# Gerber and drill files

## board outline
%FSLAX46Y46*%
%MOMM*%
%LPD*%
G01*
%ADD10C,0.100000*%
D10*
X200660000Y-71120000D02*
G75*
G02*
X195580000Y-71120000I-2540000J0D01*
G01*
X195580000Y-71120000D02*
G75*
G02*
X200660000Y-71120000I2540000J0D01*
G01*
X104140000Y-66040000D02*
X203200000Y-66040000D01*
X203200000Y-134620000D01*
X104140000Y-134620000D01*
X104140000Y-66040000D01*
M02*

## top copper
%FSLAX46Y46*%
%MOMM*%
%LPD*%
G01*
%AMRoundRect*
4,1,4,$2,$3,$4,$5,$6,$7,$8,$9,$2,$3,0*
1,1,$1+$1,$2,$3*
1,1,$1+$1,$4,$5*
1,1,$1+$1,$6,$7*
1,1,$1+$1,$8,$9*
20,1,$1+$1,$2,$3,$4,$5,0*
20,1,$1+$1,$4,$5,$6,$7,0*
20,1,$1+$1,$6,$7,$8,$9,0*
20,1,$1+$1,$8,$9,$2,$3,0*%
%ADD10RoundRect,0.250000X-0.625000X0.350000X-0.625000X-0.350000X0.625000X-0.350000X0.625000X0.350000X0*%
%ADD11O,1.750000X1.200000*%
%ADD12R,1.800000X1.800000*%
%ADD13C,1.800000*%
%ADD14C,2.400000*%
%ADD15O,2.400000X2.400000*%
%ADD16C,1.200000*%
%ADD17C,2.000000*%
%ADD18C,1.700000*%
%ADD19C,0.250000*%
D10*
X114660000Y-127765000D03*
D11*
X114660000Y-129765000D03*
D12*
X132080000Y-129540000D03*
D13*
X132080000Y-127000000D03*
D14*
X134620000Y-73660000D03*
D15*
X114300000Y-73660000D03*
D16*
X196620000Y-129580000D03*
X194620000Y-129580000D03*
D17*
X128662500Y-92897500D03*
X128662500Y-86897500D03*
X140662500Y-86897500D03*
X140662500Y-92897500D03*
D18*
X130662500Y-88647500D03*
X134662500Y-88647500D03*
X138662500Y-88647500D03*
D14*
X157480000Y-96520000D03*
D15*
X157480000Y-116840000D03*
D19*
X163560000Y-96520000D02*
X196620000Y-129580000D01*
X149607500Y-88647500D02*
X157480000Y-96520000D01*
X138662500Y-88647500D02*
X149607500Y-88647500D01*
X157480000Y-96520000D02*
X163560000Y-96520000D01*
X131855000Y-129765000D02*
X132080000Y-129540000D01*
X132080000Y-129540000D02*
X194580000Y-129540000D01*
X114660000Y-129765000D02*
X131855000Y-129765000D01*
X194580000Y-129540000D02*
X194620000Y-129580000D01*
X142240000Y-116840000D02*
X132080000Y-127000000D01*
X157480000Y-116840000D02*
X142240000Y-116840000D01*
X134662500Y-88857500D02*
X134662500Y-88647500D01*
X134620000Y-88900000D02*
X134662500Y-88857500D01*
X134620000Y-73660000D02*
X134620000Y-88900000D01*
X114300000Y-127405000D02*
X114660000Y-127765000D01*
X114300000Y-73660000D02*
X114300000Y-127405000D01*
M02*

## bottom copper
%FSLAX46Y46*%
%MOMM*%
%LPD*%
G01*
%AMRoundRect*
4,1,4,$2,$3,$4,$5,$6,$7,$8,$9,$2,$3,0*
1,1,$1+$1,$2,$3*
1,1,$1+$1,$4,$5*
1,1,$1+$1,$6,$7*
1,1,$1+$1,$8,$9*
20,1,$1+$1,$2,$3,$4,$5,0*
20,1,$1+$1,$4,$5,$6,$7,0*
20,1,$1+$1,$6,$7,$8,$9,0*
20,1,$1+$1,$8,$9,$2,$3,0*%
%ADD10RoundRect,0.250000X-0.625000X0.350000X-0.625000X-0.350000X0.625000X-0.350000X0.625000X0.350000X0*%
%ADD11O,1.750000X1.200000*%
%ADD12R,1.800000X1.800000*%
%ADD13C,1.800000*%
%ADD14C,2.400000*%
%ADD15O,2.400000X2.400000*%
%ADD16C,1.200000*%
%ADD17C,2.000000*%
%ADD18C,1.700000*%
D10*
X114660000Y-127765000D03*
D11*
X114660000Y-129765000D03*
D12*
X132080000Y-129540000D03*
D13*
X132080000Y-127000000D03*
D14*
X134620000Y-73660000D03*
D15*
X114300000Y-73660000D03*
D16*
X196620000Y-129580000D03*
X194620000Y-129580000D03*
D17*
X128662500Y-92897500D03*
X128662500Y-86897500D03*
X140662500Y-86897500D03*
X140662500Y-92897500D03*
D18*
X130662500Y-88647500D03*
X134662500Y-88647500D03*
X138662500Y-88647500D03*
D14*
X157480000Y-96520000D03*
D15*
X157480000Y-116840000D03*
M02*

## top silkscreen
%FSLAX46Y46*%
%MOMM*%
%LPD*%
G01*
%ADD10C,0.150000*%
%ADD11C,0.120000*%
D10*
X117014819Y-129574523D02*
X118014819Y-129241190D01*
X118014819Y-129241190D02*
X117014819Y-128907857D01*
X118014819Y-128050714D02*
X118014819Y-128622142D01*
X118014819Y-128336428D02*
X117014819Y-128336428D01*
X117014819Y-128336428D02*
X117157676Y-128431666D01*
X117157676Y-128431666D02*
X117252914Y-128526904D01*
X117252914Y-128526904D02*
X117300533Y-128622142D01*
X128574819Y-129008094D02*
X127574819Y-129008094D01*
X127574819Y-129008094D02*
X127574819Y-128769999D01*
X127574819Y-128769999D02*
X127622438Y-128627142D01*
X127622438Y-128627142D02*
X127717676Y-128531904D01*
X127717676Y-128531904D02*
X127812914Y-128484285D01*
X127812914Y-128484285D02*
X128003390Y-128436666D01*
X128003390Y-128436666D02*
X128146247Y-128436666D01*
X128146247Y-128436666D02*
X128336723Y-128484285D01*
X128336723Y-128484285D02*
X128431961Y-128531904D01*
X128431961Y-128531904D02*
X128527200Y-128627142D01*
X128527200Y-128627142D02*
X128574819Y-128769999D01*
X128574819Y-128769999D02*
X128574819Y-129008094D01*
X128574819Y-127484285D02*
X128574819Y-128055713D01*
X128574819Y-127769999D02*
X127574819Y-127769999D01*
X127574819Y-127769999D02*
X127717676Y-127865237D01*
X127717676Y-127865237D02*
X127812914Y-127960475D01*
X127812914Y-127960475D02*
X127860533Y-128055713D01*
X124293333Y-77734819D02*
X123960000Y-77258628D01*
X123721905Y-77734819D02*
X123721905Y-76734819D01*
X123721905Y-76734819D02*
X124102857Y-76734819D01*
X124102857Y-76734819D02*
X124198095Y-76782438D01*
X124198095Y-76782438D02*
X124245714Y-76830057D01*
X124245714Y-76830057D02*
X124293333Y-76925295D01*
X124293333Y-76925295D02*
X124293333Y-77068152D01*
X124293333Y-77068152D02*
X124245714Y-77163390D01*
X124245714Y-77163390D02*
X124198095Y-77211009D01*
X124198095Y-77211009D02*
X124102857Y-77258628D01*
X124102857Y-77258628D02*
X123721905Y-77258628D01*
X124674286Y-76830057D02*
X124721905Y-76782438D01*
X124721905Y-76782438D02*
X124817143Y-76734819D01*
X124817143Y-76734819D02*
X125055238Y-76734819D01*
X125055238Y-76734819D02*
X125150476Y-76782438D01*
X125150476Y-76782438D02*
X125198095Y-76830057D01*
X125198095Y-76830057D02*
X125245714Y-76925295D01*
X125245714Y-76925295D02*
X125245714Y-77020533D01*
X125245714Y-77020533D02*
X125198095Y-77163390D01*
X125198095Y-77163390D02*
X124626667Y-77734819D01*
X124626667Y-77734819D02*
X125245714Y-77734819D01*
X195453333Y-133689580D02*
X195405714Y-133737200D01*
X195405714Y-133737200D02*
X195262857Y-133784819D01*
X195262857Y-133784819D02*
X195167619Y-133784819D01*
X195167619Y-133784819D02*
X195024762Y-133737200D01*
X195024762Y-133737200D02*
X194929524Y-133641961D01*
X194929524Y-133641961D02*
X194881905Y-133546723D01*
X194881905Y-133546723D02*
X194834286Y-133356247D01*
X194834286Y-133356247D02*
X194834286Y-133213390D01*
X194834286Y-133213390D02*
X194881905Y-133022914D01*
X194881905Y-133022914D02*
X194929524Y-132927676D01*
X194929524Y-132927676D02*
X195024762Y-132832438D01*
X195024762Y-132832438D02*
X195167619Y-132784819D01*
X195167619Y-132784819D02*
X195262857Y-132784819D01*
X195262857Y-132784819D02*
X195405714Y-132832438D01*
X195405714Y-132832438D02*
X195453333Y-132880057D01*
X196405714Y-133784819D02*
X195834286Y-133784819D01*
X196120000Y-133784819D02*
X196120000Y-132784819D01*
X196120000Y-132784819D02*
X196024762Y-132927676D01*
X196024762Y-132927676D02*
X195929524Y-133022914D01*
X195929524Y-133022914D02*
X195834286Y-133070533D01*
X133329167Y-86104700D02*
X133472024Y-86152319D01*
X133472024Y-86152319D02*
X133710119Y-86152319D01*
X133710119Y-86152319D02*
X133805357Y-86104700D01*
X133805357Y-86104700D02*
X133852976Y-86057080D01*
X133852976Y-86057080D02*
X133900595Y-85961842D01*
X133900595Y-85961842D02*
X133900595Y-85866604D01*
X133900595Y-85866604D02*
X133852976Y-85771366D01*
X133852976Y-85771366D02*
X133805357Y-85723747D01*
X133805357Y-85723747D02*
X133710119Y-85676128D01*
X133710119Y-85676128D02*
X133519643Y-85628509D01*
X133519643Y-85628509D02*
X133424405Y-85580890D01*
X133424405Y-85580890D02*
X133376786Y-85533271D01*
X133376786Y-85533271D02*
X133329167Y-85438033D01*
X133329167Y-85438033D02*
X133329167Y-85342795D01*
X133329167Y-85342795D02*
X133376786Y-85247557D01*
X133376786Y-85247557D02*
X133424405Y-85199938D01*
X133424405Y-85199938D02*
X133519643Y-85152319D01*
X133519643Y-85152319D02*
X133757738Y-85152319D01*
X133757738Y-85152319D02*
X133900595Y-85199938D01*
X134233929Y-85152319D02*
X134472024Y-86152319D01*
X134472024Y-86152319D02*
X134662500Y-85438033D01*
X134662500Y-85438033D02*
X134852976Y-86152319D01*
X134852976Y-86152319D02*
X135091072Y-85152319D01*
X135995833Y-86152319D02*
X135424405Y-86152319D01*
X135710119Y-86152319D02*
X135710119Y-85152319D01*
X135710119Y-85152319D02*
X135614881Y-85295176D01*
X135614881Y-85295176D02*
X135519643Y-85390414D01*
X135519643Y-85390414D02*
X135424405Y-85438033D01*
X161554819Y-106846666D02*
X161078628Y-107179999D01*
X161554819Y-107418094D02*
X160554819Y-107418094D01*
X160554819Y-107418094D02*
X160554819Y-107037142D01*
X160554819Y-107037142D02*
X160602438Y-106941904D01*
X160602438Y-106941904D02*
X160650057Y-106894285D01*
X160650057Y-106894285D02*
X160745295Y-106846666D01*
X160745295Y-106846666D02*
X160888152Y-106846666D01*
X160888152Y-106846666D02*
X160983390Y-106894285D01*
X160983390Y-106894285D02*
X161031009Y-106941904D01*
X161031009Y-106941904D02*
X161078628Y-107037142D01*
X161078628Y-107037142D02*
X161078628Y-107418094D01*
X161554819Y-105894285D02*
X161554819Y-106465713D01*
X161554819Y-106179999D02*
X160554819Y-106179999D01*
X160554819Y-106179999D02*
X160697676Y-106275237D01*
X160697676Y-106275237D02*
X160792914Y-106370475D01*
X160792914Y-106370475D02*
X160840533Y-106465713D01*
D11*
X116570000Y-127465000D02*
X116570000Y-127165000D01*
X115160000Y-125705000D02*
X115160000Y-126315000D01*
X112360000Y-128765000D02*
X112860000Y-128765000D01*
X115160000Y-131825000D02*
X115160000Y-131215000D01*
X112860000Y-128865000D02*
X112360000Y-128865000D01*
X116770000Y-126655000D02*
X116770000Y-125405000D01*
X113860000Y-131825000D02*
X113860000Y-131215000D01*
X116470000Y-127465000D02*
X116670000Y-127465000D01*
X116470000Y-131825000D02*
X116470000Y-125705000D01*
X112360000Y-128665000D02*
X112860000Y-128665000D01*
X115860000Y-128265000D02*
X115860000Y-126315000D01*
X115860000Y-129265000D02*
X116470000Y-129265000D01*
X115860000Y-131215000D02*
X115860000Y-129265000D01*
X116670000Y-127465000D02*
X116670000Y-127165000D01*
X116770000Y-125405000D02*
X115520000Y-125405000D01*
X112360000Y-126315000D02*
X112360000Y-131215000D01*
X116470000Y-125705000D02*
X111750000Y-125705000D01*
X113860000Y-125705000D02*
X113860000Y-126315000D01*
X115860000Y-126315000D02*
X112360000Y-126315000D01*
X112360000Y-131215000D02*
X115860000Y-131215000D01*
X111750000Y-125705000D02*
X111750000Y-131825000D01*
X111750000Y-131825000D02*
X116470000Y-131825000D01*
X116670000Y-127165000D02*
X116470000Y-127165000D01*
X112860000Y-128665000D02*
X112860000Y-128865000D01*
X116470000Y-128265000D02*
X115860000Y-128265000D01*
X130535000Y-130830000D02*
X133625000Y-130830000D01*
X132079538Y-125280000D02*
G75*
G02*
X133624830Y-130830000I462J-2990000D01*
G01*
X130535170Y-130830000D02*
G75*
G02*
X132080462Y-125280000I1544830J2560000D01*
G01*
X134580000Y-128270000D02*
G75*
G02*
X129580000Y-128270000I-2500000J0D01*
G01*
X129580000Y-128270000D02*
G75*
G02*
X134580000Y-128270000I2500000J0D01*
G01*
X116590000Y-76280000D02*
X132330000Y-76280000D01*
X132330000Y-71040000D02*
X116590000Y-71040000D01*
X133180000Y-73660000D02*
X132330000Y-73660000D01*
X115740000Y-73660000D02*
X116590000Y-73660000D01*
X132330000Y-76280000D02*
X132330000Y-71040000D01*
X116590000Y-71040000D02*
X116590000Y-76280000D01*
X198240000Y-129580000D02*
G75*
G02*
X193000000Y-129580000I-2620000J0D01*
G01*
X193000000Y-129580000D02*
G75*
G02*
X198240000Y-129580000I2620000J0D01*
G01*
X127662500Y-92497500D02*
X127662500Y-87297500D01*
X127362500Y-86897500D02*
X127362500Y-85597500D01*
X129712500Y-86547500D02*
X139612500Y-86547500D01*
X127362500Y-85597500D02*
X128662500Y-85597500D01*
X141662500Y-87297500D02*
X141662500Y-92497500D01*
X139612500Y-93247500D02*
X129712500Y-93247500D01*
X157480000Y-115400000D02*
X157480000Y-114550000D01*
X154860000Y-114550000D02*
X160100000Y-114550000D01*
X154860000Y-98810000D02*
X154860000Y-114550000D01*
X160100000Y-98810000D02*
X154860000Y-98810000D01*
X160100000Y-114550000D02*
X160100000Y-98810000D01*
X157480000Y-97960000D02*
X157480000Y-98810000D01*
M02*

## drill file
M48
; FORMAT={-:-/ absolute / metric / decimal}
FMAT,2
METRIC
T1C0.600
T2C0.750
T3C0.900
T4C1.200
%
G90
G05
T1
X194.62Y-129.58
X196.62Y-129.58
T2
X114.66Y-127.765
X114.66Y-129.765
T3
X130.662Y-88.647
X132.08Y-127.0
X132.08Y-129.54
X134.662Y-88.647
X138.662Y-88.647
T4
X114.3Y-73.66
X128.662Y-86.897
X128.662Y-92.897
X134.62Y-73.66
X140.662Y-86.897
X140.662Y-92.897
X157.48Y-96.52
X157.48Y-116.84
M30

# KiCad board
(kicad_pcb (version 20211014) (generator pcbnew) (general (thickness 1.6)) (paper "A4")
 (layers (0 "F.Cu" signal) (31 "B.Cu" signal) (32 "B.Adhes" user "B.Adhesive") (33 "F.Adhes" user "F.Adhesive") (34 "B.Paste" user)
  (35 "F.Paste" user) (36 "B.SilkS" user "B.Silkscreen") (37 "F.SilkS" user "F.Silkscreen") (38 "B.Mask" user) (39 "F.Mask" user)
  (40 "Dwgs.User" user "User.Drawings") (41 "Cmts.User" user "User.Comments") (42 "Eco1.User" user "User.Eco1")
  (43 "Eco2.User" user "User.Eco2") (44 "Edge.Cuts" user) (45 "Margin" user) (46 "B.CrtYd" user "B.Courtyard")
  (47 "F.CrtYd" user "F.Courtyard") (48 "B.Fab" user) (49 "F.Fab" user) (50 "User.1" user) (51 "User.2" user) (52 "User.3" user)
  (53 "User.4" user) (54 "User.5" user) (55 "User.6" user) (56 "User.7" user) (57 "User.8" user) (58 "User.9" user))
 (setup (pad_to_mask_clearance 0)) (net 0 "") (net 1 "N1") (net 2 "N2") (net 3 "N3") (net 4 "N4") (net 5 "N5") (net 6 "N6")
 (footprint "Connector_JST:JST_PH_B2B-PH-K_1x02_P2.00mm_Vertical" (layer "F.Cu") (at 114.66 127.765 -90)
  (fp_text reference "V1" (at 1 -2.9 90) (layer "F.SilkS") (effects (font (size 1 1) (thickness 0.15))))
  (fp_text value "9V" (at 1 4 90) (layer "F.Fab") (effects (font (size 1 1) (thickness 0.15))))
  (fp_line (start -0.3 -1.91) (end -0.6 -1.91) (layer "F.SilkS") (width 0.12))
  (fp_line (start -2.06 -0.5) (end -1.45 -0.5) (layer "F.SilkS") (width 0.12))
  (fp_line (start 1 2.3) (end 1 1.8) (layer "F.SilkS") (width 0.12))
  (fp_line (start 4.06 -0.5) (end 3.45 -0.5) (layer "F.SilkS") (width 0.12))
  (fp_line (start 1.1 1.8) (end 1.1 2.3) (layer "F.SilkS") (width 0.12))
  (fp_line (start -1.11 -2.11) (end -2.36 -2.11) (layer "F.SilkS") (width 0.12))
  (fp_line (start 4.06 0.8) (end 3.45 0.8) (layer "F.SilkS") (width 0.12))
  (fp_line (start -0.3 -1.81) (end -0.3 -2.01) (layer "F.SilkS") (width 0.12))
  (fp_line (start 4.06 -1.81) (end -2.06 -1.81) (layer "F.SilkS") (width 0.12))
  (fp_line (start 0.9 2.3) (end 0.9 1.8) (layer "F.SilkS") (width 0.12))
  (fp_line (start 0.5 -1.2) (end -1.45 -1.2) (layer "F.SilkS") (width 0.12))
  (fp_line (start 1.5 -1.2) (end 1.5 -1.81) (layer "F.SilkS") (width 0.12))
  (fp_line (start 3.45 -1.2) (end 1.5 -1.2) (layer "F.SilkS") (width 0.12))
  (fp_line (start -0.3 -2.01) (end -0.6 -2.01) (layer "F.SilkS") (width 0.12))
  (fp_line (start -2.36 -2.11) (end -2.36 -0.86) (layer "F.SilkS") (width 0.12))
  (fp_line (start -1.45 2.3) (end 3.45 2.3) (layer "F.SilkS") (width 0.12))
  (fp_line (start -2.06 -1.81) (end -2.06 2.91) (layer "F.SilkS") (width 0.12))
  (fp_line (start -2.06 0.8) (end -1.45 0.8) (layer "F.SilkS") (width 0.12))
  (fp_line (start -1.45 -1.2) (end -1.45 2.3) (layer "F.SilkS") (width 0.12))
  (fp_line (start 3.45 2.3) (end 3.45 -1.2) (layer "F.SilkS") (width 0.12))
  (fp_line (start -2.06 2.91) (end 4.06 2.91) (layer "F.SilkS") (width 0.12))
  (fp_line (start 4.06 2.91) (end 4.06 -1.81) (layer "F.SilkS") (width 0.12))
  (fp_line (start -0.6 -2.01) (end -0.6 -1.81) (layer "F.SilkS") (width 0.12))
  (fp_line (start 0.9 1.8) (end 1.1 1.8) (layer "F.SilkS") (width 0.12))
  (fp_line (start 0.5 -1.81) (end 0.5 -1.2) (layer "F.SilkS") (width 0.12))
  (pad "1" thru_hole roundrect (at 0 0 270) (size 1.2 1.75) (drill 0.75) (layers *.Cu *.Mask) (roundrect_rratio 0.208333) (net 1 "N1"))
  (pad "2" thru_hole oval (at 2 0 270) (size 1.2 1.75) (drill 0.75) (layers *.Cu *.Mask) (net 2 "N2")))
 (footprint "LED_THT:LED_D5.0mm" (layer "F.Cu") (at 132.08 129.54 90)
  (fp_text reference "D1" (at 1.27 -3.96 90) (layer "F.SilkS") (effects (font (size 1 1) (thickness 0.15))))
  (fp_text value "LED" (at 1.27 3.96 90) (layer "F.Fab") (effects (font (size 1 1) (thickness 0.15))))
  (fp_line (start -1.29 -1.545) (end -1.29 1.545) (layer "F.SilkS") (width 0.12))
  (fp_arc (start 4.26 -0.000462) (mid 2.072002 2.880433) (end -1.29 1.54483) (layer "F.SilkS") (width 0.12))
  (fp_arc (start -1.29 -1.54483) (mid 2.072002 -2.880433) (end 4.26 0.000462) (layer "F.SilkS") (width 0.12))
  (fp_circle (center 1.27 0) (end 3.77 0) (layer "F.SilkS") (width 0.12) (fill none))
  (pad "1" thru_hole rect (at 0 0 90) (size 1.8 1.8) (drill 0.9) (layers *.Cu *.Mask) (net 2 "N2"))
  (pad "2" thru_hole circle (at 2.54 0 90) (size 1.8 1.8) (drill 0.9) (layers *.Cu *.Mask) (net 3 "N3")))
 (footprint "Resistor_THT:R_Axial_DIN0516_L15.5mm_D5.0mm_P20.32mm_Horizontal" (layer "F.Cu") (at 134.62 73.66 180)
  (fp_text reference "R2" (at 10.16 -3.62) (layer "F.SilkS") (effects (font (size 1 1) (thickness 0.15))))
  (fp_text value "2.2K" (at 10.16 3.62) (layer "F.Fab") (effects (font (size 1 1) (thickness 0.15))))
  (fp_line (start 18.03 -2.62) (end 2.29 -2.62) (layer "F.SilkS") (width 0.12))
  (fp_line (start 2.29 2.62) (end 18.03 2.62) (layer "F.SilkS") (width 0.12))
  (fp_line (start 1.44 0) (end 2.29 0) (layer "F.SilkS") (width 0.12))
  (fp_line (start 18.88 0) (end 18.03 0) (layer "F.SilkS") (width 0.12))
  (fp_line (start 2.29 -2.62) (end 2.29 2.62) (layer "F.SilkS") (width 0.12))
  (fp_line (start 18.03 2.62) (end 18.03 -2.62) (layer "F.SilkS") (width 0.12))
  (pad "1" thru_hole circle (at 0 0 180) (size 2.4 2.4) (drill 1.2) (layers *.Cu *.Mask) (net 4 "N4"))
  (pad "2" thru_hole oval (at 20.32 0 180) (size 2.4 2.4) (drill 1.2) (layers *.Cu *.Mask) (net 1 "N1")))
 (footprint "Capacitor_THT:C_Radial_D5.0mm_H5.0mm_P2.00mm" (layer "F.Cu") (at 196.62 129.58 180)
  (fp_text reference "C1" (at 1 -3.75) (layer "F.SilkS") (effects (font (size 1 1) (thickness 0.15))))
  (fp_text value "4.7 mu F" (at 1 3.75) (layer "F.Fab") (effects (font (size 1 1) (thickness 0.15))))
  (fp_circle (center 1 0) (end 3.62 0) (layer "F.SilkS") (width 0.12) (fill none))
  (pad "1" thru_hole circle (at 0 0 180) (size 1.2 1.2) (drill 0.6) (layers *.Cu *.Mask) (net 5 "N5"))
  (pad "2" thru_hole circle (at 2 0 180) (size 1.2 1.2) (drill 0.6) (layers *.Cu *.Mask) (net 2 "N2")))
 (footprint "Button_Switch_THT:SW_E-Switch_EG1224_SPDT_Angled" (layer "F.Cu") (at 130.6625 88.6475)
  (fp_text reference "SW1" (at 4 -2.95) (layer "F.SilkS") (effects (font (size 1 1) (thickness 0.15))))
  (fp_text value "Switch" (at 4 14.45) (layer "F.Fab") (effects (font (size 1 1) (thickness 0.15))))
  (fp_line (start -3 3.85) (end -3 -1.35) (layer "F.SilkS") (width 0.12))
  (fp_line (start -3.3 -1.75) (end -3.3 -3.05) (layer "F.SilkS") (width 0.12))
  (fp_line (start -0.95 -2.1) (end 8.95 -2.1) (layer "F.SilkS") (width 0.12))
  (fp_line (start -3.3 -3.05) (end -2 -3.05) (layer "F.SilkS") (width 0.12))
  (fp_line (start 11 -1.35) (end 11 3.85) (layer "F.SilkS") (width 0.12))
  (fp_line (start 8.95 4.6) (end -0.95 4.6) (layer "F.SilkS") (width 0.12))
  (pad "" thru_hole circle (at -2 4.25) (size 2 2) (drill 1.2) (layers *.Cu *.Mask))
  (pad "" thru_hole circle (at -2 -1.75) (size 2 2) (drill 1.2) (layers *.Cu *.Mask))
  (pad "" thru_hole circle (at 10 -1.75) (size 2 2) (drill 1.2) (layers *.Cu *.Mask))
  (pad "" thru_hole circle (at 10 4.25) (size 2 2) (drill 1.2) (layers *.Cu *.Mask))
  (pad "1" thru_hole circle (at 0 0) (size 1.7 1.7) (drill 0.9) (layers *.Cu *.Mask) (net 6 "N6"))
  (pad "2" thru_hole circle (at 4 0) (size 1.7 1.7) (drill 0.9) (layers *.Cu *.Mask) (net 4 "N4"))
  (pad "3" thru_hole circle (at 8 0) (size 1.7 1.7) (drill 0.9) (layers *.Cu *.Mask) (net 5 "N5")))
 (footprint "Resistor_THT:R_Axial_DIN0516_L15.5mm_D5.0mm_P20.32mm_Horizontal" (layer "F.Cu") (at 157.48 96.52 -90)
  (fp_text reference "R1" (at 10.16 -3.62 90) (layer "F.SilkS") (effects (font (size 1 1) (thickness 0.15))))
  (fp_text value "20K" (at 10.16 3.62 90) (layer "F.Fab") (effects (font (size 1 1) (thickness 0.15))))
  (fp_line (start 18.88 0) (end 18.03 0) (layer "F.SilkS") (width 0.12))
  (fp_line (start 18.03 2.62) (end 18.03 -2.62) (layer "F.SilkS") (width 0.12))
  (fp_line (start 2.29 2.62) (end 18.03 2.62) (layer "F.SilkS") (width 0.12))
  (fp_line (start 2.29 -2.62) (end 2.29 2.62) (layer "F.SilkS") (width 0.12))
  (fp_line (start 18.03 -2.62) (end 2.29 -2.62) (layer "F.SilkS") (width 0.12))
  (fp_line (start 1.44 0) (end 2.29 0) (layer "F.SilkS") (width 0.12))
  (pad "1" thru_hole circle (at 0 0 270) (size 2.4 2.4) (drill 1.2) (layers *.Cu *.Mask) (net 5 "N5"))
  (pad "2" thru_hole oval (at 20.32 0 270) (size 2.4 2.4) (drill 1.2) (layers *.Cu *.Mask) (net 3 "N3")))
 (gr_circle (center 198.12 71.12) (end 198.12 73.66) (layer "Edge.Cuts") (width 0.1) (fill none))
 (gr_rect (start 104.14 66.04) (end 203.2 134.62) (layer "Edge.Cuts") (width 0.1) (fill none))
 (segment (start 163.56 96.52) (end 196.62 129.58) (width 0.25) (layer "F.Cu") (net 5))
 (segment (start 149.6075 88.6475) (end 157.48 96.52) (width 0.25) (layer "F.Cu") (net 5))
 (segment (start 138.6625 88.6475) (end 149.6075 88.6475) (width 0.25) (layer "F.Cu") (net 5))
 (segment (start 157.48 96.52) (end 163.56 96.52) (width 0.25) (layer "F.Cu") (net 5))
 (segment (start 131.855 129.765) (end 132.08 129.54) (width 0.25) (layer "F.Cu") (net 2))
 (segment (start 132.08 129.54) (end 194.58 129.54) (width 0.25) (layer "F.Cu") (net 2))
 (segment (start 114.66 129.765) (end 131.855 129.765) (width 0.25) (layer "F.Cu") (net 2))
 (segment (start 194.58 129.54) (end 194.62 129.58) (width 0.25) (layer "F.Cu") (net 2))
 (segment (start 142.24 116.84) (end 132.08 127) (width 0.25) (layer "F.Cu") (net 3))
 (segment (start 157.48 116.84) (end 142.24 116.84) (width 0.25) (layer "F.Cu") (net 3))
 (segment (start 134.6625 88.8575) (end 134.6625 88.6475) (width 0.25) (layer "F.Cu") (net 4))
 (segment (start 134.62 88.9) (end 134.6625 88.8575) (width 0.25) (layer "F.Cu") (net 4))
 (segment (start 134.62 73.66) (end 134.62 88.9) (width 0.25) (layer "F.Cu") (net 4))
 (segment (start 114.3 127.405) (end 114.66 127.765) (width 0.25) (layer "F.Cu") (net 1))
 (segment (start 114.3 73.66) (end 114.3 127.405) (width 0.25) (layer "F.Cu") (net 1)))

